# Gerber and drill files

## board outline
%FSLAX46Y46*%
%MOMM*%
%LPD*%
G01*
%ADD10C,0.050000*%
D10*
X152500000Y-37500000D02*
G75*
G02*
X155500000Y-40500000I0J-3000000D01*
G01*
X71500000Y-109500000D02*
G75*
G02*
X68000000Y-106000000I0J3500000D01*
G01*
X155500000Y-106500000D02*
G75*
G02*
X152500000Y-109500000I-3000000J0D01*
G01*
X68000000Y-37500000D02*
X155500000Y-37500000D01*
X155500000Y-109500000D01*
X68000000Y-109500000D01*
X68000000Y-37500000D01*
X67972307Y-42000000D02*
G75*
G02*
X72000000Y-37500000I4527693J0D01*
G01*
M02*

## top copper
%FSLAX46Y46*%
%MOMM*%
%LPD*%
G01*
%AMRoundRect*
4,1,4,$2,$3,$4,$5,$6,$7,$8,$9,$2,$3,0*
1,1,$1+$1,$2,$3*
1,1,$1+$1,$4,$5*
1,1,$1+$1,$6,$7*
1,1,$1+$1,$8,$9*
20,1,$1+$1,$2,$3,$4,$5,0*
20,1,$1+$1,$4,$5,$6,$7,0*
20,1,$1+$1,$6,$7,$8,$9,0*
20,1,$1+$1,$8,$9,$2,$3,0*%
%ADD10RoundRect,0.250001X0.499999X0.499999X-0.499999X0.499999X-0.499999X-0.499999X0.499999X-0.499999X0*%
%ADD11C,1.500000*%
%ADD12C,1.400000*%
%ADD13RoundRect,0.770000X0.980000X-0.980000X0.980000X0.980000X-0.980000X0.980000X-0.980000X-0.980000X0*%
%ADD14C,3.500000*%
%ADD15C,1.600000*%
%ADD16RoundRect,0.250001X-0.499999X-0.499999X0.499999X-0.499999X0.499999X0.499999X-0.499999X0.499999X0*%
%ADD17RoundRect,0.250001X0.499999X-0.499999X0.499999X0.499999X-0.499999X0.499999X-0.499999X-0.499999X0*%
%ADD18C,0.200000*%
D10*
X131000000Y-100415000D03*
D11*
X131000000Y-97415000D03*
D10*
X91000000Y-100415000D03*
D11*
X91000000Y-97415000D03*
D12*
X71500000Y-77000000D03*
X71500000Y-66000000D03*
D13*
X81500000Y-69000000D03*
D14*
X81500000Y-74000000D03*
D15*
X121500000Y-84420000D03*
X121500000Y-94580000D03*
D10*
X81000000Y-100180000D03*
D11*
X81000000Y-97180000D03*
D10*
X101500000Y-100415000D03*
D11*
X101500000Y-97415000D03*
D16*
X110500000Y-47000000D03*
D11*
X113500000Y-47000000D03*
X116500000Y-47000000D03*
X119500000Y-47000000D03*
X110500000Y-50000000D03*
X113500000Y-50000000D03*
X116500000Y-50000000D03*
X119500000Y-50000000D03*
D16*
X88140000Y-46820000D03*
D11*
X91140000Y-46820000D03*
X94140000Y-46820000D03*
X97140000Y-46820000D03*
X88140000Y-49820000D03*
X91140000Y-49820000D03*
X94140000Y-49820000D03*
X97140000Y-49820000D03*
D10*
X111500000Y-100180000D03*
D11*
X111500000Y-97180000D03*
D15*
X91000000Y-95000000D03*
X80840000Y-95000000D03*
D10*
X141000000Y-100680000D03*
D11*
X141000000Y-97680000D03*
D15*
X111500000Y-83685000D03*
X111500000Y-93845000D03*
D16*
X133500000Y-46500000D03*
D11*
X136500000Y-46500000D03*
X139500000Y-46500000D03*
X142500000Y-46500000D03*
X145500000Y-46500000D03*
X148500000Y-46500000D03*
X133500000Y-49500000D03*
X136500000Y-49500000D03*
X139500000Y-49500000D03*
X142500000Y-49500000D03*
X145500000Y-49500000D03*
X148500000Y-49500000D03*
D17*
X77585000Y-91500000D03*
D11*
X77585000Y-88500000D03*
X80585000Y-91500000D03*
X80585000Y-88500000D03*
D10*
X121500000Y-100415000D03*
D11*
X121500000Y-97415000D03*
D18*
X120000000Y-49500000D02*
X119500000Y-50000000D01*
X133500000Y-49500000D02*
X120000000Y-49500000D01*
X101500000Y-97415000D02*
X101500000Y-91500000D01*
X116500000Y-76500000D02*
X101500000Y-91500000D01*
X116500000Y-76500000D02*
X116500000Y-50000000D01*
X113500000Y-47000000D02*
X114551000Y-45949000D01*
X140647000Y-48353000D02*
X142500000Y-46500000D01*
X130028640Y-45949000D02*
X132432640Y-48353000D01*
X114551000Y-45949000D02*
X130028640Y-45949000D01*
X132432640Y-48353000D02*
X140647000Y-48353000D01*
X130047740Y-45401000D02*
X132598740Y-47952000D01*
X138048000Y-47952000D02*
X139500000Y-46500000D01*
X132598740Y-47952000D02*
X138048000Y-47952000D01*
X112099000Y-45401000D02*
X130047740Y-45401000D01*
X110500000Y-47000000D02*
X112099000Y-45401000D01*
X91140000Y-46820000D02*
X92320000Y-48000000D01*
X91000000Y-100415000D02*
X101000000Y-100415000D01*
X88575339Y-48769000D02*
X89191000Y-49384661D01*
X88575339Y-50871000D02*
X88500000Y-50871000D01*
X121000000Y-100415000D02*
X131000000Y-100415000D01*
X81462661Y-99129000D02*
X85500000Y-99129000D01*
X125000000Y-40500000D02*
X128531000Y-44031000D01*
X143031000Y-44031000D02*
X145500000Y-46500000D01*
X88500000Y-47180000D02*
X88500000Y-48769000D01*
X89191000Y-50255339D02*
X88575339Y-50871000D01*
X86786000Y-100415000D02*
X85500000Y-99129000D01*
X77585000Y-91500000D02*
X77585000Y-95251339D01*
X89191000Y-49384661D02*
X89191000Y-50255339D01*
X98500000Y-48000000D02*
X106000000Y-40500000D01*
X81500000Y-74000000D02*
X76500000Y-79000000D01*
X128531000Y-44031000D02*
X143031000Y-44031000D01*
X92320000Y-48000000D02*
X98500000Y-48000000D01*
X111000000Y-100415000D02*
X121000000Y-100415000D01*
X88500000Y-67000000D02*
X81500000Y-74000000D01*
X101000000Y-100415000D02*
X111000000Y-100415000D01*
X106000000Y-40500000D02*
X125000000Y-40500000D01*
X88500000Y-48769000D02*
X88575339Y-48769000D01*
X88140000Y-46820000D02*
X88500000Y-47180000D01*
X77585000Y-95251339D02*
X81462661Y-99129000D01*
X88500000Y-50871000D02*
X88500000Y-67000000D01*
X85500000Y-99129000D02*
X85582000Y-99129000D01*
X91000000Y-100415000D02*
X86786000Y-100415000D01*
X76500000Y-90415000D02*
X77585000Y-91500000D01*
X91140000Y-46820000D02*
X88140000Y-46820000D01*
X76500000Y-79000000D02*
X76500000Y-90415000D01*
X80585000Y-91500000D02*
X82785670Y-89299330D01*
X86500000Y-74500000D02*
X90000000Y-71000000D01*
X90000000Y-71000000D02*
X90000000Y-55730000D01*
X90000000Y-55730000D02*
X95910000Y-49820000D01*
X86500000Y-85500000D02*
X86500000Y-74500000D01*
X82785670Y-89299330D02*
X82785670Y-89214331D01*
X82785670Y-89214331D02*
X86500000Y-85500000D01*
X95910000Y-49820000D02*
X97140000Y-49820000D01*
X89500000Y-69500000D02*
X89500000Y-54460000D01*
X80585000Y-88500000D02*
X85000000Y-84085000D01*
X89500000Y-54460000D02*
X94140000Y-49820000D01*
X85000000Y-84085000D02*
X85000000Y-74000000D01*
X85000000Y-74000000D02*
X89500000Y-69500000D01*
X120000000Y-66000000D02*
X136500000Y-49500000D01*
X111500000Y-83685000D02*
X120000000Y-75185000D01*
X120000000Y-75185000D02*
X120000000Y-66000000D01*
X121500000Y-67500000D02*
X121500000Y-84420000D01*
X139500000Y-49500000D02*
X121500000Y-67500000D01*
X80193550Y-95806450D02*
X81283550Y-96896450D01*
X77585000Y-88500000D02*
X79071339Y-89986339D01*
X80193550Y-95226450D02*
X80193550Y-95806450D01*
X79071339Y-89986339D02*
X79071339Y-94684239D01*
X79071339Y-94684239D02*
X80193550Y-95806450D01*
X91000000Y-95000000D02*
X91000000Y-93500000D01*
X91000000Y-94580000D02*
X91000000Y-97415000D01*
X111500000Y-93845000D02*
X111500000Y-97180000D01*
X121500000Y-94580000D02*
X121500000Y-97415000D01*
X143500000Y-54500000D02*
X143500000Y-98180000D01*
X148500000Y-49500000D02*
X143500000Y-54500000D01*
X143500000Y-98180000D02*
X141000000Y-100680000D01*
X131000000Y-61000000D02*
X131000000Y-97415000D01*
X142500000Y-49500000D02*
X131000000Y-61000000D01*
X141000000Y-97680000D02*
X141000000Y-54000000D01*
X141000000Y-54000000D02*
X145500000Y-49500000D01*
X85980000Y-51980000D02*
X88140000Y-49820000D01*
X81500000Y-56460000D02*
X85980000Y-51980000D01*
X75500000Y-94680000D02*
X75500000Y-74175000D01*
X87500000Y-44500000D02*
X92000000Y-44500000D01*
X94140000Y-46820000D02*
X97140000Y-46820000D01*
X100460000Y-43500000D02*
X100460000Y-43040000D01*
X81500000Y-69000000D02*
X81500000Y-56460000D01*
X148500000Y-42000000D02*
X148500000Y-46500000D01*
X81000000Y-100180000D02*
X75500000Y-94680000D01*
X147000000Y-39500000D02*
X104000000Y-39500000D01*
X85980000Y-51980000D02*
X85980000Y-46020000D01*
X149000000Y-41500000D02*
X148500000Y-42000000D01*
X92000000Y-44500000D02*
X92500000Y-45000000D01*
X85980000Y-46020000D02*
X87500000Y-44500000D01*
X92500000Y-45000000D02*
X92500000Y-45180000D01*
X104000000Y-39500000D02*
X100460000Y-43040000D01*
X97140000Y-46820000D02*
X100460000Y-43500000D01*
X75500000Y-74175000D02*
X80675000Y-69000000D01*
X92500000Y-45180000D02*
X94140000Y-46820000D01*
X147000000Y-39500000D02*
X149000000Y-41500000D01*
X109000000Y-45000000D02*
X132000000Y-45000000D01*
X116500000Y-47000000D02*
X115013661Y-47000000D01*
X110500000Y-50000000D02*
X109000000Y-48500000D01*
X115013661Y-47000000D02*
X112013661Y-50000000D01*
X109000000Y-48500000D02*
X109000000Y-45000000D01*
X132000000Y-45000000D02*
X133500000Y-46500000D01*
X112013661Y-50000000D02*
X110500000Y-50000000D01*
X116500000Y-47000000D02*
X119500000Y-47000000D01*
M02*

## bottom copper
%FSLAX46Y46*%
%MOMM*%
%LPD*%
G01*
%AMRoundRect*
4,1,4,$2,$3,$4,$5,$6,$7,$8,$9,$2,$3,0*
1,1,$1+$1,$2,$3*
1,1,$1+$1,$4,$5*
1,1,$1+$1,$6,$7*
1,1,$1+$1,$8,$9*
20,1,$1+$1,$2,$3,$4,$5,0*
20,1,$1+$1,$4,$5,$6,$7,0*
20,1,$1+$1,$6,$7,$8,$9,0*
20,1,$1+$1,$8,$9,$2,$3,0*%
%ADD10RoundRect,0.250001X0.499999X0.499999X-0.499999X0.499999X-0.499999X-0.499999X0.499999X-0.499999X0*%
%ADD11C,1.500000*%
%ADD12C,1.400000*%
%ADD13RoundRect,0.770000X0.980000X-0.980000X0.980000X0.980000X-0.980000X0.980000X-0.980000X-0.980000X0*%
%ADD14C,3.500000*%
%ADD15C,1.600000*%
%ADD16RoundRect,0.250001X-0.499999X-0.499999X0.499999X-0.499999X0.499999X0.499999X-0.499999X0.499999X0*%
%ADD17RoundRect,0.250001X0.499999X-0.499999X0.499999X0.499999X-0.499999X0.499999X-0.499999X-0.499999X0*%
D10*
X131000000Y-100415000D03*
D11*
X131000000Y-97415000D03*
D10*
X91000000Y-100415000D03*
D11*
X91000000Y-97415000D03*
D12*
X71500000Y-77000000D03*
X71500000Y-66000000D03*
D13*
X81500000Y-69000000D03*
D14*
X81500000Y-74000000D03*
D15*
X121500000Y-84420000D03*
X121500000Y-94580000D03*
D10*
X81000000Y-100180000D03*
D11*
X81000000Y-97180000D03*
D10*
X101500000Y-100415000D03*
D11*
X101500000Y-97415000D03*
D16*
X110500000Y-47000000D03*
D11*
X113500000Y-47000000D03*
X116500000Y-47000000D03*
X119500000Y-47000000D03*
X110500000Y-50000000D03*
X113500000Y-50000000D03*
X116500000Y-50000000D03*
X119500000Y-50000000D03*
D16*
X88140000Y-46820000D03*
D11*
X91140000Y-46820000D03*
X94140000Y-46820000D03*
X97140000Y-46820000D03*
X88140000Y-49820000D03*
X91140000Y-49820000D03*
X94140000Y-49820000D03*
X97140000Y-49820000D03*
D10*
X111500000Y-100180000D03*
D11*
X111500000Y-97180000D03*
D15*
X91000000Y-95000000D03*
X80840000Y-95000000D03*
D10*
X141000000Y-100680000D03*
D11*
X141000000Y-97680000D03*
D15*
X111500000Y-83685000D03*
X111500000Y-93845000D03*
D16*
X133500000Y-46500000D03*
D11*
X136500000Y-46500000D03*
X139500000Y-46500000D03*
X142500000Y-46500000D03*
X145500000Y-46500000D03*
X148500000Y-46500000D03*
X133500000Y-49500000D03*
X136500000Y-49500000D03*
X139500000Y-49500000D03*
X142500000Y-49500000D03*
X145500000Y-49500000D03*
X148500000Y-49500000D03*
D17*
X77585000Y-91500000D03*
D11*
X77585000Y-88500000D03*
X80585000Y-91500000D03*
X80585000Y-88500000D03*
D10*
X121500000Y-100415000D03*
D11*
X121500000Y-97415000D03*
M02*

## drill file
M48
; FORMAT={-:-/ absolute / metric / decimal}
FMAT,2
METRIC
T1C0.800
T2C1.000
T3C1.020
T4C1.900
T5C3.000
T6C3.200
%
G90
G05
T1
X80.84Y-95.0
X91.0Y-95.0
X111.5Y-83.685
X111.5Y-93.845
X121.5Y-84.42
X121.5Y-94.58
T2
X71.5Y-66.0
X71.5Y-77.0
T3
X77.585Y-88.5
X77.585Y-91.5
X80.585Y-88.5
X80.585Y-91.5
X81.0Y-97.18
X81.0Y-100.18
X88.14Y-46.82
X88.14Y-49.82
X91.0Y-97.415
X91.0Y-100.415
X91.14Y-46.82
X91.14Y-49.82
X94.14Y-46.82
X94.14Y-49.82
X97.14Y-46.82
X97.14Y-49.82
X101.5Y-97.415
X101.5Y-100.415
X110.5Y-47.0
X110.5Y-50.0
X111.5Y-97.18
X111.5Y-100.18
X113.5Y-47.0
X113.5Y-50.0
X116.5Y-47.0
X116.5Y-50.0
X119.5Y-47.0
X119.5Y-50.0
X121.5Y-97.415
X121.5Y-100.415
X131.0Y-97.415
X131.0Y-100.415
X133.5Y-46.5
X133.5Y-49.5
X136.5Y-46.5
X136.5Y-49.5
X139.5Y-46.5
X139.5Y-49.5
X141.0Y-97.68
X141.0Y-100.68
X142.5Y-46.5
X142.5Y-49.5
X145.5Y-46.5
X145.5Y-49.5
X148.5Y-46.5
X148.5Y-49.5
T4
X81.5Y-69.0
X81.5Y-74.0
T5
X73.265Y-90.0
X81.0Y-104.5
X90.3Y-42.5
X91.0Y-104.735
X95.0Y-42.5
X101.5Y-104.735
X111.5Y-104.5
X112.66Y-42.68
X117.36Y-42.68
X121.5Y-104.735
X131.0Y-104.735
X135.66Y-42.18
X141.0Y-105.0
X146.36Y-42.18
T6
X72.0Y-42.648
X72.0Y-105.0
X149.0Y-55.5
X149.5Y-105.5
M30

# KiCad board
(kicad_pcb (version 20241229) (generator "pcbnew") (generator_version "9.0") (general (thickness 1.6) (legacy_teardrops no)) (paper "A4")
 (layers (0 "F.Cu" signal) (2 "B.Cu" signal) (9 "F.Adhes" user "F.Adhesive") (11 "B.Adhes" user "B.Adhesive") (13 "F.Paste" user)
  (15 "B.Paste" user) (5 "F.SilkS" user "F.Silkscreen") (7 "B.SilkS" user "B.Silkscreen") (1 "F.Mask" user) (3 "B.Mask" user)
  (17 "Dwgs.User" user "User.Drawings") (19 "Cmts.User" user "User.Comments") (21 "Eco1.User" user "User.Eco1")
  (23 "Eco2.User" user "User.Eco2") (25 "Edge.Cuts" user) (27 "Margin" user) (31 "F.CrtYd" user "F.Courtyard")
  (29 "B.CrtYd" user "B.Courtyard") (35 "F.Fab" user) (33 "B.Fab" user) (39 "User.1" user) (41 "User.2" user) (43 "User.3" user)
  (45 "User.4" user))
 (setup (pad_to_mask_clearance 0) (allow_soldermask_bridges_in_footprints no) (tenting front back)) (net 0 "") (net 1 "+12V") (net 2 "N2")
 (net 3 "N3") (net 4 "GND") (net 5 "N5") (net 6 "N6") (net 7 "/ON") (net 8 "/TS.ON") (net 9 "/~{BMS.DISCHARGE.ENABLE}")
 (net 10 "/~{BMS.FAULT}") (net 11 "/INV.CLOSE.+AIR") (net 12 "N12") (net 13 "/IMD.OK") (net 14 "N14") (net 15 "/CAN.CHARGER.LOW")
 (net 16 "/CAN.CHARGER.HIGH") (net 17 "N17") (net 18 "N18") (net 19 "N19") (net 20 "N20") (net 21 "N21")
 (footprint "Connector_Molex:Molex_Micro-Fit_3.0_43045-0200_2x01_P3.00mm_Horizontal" (layer "F.Cu") (at 131 100.415 180)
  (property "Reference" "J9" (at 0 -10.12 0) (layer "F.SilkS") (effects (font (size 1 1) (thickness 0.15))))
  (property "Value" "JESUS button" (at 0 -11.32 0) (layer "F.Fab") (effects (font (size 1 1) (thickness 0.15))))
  (pad "" np_thru_hole circle (at 0 -4.32 180) (size 3 3) (drill 3) (layers "*.Cu" "*.Mask"))
  (pad "1" thru_hole roundrect (at 0 0 180) (size 1.5 1.5) (drill 1.02) (layers "*.Cu" "*.Mask") (remove_unused_layers no)
   (roundrect_rratio 0.166667) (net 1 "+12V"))
  (pad "2" thru_hole circle (at 0 3 180) (size 1.5 1.5) (drill 1.02) (layers "*.Cu" "*.Mask") (remove_unused_layers no) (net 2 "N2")))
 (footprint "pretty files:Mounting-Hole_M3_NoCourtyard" (layer "F.Cu") (at 150.41 110.58)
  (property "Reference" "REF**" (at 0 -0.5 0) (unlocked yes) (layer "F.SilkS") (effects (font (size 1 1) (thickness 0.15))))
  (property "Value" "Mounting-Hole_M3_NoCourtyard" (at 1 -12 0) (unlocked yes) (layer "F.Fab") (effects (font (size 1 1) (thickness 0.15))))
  (pad "" np_thru_hole circle (at -0.91 -5.08) (size 3.2 3.2) (drill 3.2) (layers "*.Cu" "*.Mask")))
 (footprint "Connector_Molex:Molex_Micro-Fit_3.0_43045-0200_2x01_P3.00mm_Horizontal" (layer "F.Cu") (at 91 100.415 180)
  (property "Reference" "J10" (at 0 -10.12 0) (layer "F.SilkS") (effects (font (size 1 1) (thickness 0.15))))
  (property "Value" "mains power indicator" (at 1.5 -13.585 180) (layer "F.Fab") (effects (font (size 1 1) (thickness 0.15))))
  (pad "" np_thru_hole circle (at 0 -4.32 180) (size 3 3) (drill 3) (layers "*.Cu" "*.Mask"))
  (pad "1" thru_hole roundrect (at 0 0 180) (size 1.5 1.5) (drill 1.02) (layers "*.Cu" "*.Mask") (remove_unused_layers no)
   (roundrect_rratio 0.166667) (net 1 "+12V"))
  (pad "2" thru_hole circle (at 0 3 180) (size 1.5 1.5) (drill 1.02) (layers "*.Cu" "*.Mask") (remove_unused_layers no) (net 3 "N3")))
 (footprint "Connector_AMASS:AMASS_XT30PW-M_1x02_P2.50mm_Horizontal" (layer "F.Cu") (at 81.5 69 90)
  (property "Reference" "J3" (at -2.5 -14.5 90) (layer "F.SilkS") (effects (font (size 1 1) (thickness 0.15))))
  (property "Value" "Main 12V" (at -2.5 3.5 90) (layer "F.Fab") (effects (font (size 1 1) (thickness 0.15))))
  (pad "" thru_hole circle (at -8 -10 90) (size 1.4 1.4) (drill 1) (layers "*.Cu" "*.Mask") (remove_unused_layers no))
  (pad "" thru_hole circle (at 3 -10 90) (size 1.4 1.4) (drill 1) (layers "*.Cu" "*.Mask") (remove_unused_layers no))
  (pad "1" thru_hole roundrect (at 0 0 90) (size 3.5 3.5) (drill 1.9) (layers "*.Cu" "*.Mask") (remove_unused_layers no)
   (roundrect_rratio 0.22) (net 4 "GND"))
  (pad "2" thru_hole circle (at -5 0 90) (size 3.5 3.5) (drill 1.9) (layers "*.Cu" "*.Mask") (remove_unused_layers no) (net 1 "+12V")))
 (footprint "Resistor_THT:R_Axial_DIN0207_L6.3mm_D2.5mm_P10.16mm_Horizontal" (layer "F.Cu") (at 121.5 84.42 -90)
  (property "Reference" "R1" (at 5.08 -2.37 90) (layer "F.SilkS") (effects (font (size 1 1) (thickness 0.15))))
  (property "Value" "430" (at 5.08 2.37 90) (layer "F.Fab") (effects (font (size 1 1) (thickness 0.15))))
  (pad "1" thru_hole circle (at 0 0 270) (size 1.6 1.6) (drill 0.8) (layers "*.Cu" "*.Mask") (remove_unused_layers no) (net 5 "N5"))
  (pad "2" thru_hole circle (at 10.16 0 270) (size 1.6 1.6) (drill 0.8) (layers "*.Cu" "*.Mask") (remove_unused_layers no) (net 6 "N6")))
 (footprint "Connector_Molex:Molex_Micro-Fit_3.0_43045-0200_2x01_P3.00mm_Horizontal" (layer "F.Cu") (at 81 100.18 180)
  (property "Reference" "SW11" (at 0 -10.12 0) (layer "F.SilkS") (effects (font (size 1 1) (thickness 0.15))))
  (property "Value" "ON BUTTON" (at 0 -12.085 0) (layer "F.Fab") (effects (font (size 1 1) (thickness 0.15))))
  (pad "" np_thru_hole circle (at 0 -4.32 180) (size 3 3) (drill 3) (layers "*.Cu" "*.Mask"))
  (pad "1" thru_hole roundrect (at 0 0 180) (size 1.5 1.5) (drill 1.02) (layers "*.Cu" "*.Mask") (remove_unused_layers no)
   (roundrect_rratio 0.166667) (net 4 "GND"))
  (pad "2" thru_hole circle (at 0 3 180) (size 1.5 1.5) (drill 1.02) (layers "*.Cu" "*.Mask") (remove_unused_layers no) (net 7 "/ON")))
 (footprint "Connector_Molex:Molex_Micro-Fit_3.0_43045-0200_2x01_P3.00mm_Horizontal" (layer "F.Cu") (at 101.5 100.415 180)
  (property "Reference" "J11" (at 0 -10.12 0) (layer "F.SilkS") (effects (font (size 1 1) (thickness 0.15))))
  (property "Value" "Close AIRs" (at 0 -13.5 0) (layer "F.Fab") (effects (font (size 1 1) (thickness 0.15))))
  (pad "" np_thru_hole circle (at 0 -4.32 180) (size 3 3) (drill 3) (layers "*.Cu" "*.Mask"))
  (pad "1" thru_hole roundrect (at 0 0 180) (size 1.5 1.5) (drill 1.02) (layers "*.Cu" "*.Mask") (remove_unused_layers no)
   (roundrect_rratio 0.166667) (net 1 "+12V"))
  (pad "2" thru_hole circle (at 0 3 180) (size 1.5 1.5) (drill 1.02) (layers "*.Cu" "*.Mask") (remove_unused_layers no) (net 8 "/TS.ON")))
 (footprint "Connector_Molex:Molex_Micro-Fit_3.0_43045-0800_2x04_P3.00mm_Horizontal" (layer "F.Cu") (at 110.5 47)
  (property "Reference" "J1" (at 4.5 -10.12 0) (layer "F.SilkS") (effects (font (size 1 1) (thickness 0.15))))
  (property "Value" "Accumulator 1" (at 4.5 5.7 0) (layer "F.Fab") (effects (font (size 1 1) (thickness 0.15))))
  (pad "" np_thru_hole circle (at 2.16 -4.32) (size 3 3) (drill 3) (layers "*.Cu" "*.Mask"))
  (pad "" np_thru_hole circle (at 6.86 -4.32) (size 3 3) (drill 3) (layers "*.Cu" "*.Mask"))
  (pad "1" thru_hole roundrect (at 0 0) (size 1.5 1.5) (drill 1.02) (layers "*.Cu" "*.Mask") (remove_unused_layers no)
   (roundrect_rratio 0.166667) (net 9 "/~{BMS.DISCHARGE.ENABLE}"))
  (pad "2" thru_hole circle (at 3 0) (size 1.5 1.5) (drill 1.02) (layers "*.Cu" "*.Mask") (remove_unused_layers no) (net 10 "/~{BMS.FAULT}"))
  (pad "3" thru_hole circle (at 6 0) (size 1.5 1.5) (drill 1.02) (layers "*.Cu" "*.Mask") (remove_unused_layers no)
   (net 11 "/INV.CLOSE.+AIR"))
  (pad "4" thru_hole circle (at 9 0) (size 1.5 1.5) (drill 1.02) (layers "*.Cu" "*.Mask") (remove_unused_layers no)
   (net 11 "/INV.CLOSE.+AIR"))
  (pad "5" thru_hole circle (at 0 3) (size 1.5 1.5) (drill 1.02) (layers "*.Cu" "*.Mask") (remove_unused_layers no)
   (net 11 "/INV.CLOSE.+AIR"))
  (pad "6" thru_hole circle (at 3 3) (size 1.5 1.5) (drill 1.02) (layers "*.Cu" "*.Mask") (remove_unused_layers no) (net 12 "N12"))
  (pad "7" thru_hole circle (at 6 3) (size 1.5 1.5) (drill 1.02) (layers "*.Cu" "*.Mask") (remove_unused_layers no) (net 8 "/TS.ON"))
  (pad "8" thru_hole circle (at 9 3) (size 1.5 1.5) (drill 1.02) (layers "*.Cu" "*.Mask") (remove_unused_layers no) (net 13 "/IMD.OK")))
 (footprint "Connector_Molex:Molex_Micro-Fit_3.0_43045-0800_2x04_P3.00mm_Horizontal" (layer "F.Cu") (at 88.14 46.82)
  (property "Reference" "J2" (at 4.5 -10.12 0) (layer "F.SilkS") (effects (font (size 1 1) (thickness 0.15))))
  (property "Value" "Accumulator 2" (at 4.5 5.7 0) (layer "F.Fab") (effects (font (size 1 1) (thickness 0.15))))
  (pad "" np_thru_hole circle (at 2.16 -4.32) (size 3 3) (drill 3) (layers "*.Cu" "*.Mask"))
  (pad "" np_thru_hole circle (at 6.86 -4.32) (size 3 3) (drill 3) (layers "*.Cu" "*.Mask"))
  (pad "1" thru_hole roundrect (at 0 0) (size 1.5 1.5) (drill 1.02) (layers "*.Cu" "*.Mask") (remove_unused_layers no)
   (roundrect_rratio 0.166667) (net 1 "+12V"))
  (pad "2" thru_hole circle (at 3 0) (size 1.5 1.5) (drill 1.02) (layers "*.Cu" "*.Mask") (remove_unused_layers no) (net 1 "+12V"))
  (pad "3" thru_hole circle (at 6 0) (size 1.5 1.5) (drill 1.02) (layers "*.Cu" "*.Mask") (remove_unused_layers no) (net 4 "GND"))
  (pad "4" thru_hole circle (at 9 0) (size 1.5 1.5) (drill 1.02) (layers "*.Cu" "*.Mask") (remove_unused_layers no) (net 4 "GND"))
  (pad "5" thru_hole circle (at 0 3) (size 1.5 1.5) (drill 1.02) (layers "*.Cu" "*.Mask") (remove_unused_layers no) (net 4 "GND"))
  (pad "6" thru_hole circle (at 3 3) (size 1.5 1.5) (drill 1.02) (layers "*.Cu" "*.Mask") (remove_unused_layers no) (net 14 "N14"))
  (pad "7" thru_hole circle (at 6 3) (size 1.5 1.5) (drill 1.02) (layers "*.Cu" "*.Mask") (remove_unused_layers no)
   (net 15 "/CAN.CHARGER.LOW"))
  (pad "8" thru_hole circle (at 9 3) (size 1.5 1.5) (drill 1.02) (layers "*.Cu" "*.Mask") (remove_unused_layers no)
   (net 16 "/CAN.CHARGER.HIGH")))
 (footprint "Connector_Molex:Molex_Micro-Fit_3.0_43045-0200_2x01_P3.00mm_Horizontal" (layer "F.Cu") (at 111.5 100.18 180)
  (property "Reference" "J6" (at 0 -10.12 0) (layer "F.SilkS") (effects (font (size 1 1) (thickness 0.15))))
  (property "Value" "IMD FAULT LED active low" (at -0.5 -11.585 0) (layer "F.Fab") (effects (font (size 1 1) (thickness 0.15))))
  (pad "" np_thru_hole circle (at 0 -4.32 180) (size 3 3) (drill 3) (layers "*.Cu" "*.Mask"))
  (pad "1" thru_hole roundrect (at 0 0 180) (size 1.5 1.5) (drill 1.02) (layers "*.Cu" "*.Mask") (remove_unused_layers no)
   (roundrect_rratio 0.166667) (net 1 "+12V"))
  (pad "2" thru_hole circle (at 0 3 180) (size 1.5 1.5) (drill 1.02) (layers "*.Cu" "*.Mask") (remove_unused_layers no) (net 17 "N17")))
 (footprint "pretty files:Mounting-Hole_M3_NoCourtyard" (layer "F.Cu") (at 149.91 60.58)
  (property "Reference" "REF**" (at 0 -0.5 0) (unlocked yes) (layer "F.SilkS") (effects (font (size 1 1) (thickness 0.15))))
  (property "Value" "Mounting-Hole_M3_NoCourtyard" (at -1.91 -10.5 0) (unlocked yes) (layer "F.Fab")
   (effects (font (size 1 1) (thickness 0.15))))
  (pad "" np_thru_hole circle (at -0.91 -5.08) (size 3.2 3.2) (drill 3.2) (layers "*.Cu" "*.Mask")))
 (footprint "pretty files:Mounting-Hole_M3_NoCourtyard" (layer "F.Cu") (at 72.91 47.7275)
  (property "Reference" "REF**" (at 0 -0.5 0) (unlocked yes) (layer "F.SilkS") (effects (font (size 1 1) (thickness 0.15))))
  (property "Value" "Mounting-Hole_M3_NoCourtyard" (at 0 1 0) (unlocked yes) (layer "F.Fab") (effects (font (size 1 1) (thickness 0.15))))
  (pad "" np_thru_hole circle (at -0.91 -5.08) (size 3.2 3.2) (drill 3.2) (layers "*.Cu" "*.Mask")))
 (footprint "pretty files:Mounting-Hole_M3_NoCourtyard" (layer "F.Cu") (at 72.91 110.08)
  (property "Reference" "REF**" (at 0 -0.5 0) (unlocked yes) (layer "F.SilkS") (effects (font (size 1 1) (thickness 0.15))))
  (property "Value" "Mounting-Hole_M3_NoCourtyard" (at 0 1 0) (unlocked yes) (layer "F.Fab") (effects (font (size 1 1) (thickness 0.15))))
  (pad "" np_thru_hole circle (at -0.91 -5.08) (size 3.2 3.2) (drill 3.2) (layers "*.Cu" "*.Mask")))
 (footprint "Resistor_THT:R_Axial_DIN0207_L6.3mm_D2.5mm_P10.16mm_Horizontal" (layer "F.Cu") (at 91 95 180)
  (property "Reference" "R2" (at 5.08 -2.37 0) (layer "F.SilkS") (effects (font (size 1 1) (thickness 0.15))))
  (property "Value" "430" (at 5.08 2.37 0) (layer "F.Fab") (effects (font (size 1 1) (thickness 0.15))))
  (pad "1" thru_hole circle (at 0 0 180) (size 1.6 1.6) (drill 0.8) (layers "*.Cu" "*.Mask") (remove_unused_layers no) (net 3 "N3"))
  (pad "2" thru_hole circle (at 10.16 0 180) (size 1.6 1.6) (drill 0.8) (layers "*.Cu" "*.Mask") (remove_unused_layers no) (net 7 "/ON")))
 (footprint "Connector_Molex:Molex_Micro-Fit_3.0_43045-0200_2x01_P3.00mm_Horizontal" (layer "F.Cu") (at 141 100.68 180)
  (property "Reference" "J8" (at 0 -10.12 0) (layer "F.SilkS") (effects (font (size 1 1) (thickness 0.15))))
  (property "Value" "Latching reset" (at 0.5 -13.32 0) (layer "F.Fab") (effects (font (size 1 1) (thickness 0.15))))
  (pad "" np_thru_hole circle (at 0 -4.32 180) (size 3 3) (drill 3) (layers "*.Cu" "*.Mask"))
  (pad "1" thru_hole roundrect (at 0 0 180) (size 1.5 1.5) (drill 1.02) (layers "*.Cu" "*.Mask") (remove_unused_layers no)
   (roundrect_rratio 0.166667) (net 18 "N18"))
  (pad "2" thru_hole circle (at 0 3 180) (size 1.5 1.5) (drill 1.02) (layers "*.Cu" "*.Mask") (remove_unused_layers no) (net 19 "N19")))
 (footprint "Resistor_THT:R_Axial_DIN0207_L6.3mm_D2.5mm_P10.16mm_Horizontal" (layer "F.Cu") (at 111.5 83.685 -90)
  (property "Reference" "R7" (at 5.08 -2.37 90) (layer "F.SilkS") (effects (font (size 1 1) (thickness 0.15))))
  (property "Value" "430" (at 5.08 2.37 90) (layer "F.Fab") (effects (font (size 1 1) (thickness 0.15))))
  (pad "1" thru_hole circle (at 0 0 270) (size 1.6 1.6) (drill 0.8) (layers "*.Cu" "*.Mask") (remove_unused_layers no) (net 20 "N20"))
  (pad "2" thru_hole circle (at 10.16 0 270) (size 1.6 1.6) (drill 0.8) (layers "*.Cu" "*.Mask") (remove_unused_layers no) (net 17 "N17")))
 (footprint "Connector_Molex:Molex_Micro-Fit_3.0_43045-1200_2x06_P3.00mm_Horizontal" (layer "F.Cu") (at 133.5 46.5)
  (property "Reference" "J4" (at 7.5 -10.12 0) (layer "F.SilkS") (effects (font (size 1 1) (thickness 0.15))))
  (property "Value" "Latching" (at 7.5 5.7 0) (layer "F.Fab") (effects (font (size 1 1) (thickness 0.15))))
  (pad "" np_thru_hole circle (at 2.16 -4.32) (size 3 3) (drill 3) (layers "*.Cu" "*.Mask"))
  (pad "" np_thru_hole circle (at 12.86 -4.32) (size 3 3) (drill 3) (layers "*.Cu" "*.Mask"))
  (pad "1" thru_hole roundrect (at 0 0) (size 1.5 1.5) (drill 1.02) (layers "*.Cu" "*.Mask") (remove_unused_layers no)
   (roundrect_rratio 0.166667) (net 11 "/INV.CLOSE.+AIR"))
  (pad "2" thru_hole circle (at 3 0) (size 1.5 1.5) (drill 1.02) (layers "*.Cu" "*.Mask") (remove_unused_layers no) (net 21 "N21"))
  (pad "3" thru_hole circle (at 6 0) (size 1.5 1.5) (drill 1.02) (layers "*.Cu" "*.Mask") (remove_unused_layers no)
   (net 9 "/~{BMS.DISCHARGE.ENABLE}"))
  (pad "4" thru_hole circle (at 9 0) (size 1.5 1.5) (drill 1.02) (layers "*.Cu" "*.Mask") (remove_unused_layers no) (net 10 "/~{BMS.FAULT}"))
  (pad "5" thru_hole circle (at 12 0) (size 1.5 1.5) (drill 1.02) (layers "*.Cu" "*.Mask") (remove_unused_layers no) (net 1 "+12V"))
  (pad "6" thru_hole circle (at 15 0) (size 1.5 1.5) (drill 1.02) (layers "*.Cu" "*.Mask") (remove_unused_layers no) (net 4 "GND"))
  (pad "7" thru_hole circle (at 0 3) (size 1.5 1.5) (drill 1.02) (layers "*.Cu" "*.Mask") (remove_unused_layers no) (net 13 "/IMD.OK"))
  (pad "8" thru_hole circle (at 3 3) (size 1.5 1.5) (drill 1.02) (layers "*.Cu" "*.Mask") (remove_unused_layers no) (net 20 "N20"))
  (pad "9" thru_hole circle (at 6 3) (size 1.5 1.5) (drill 1.02) (layers "*.Cu" "*.Mask") (remove_unused_layers no) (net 5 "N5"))
  (pad "10" thru_hole circle (at 9 3) (size 1.5 1.5) (drill 1.02) (layers "*.Cu" "*.Mask") (remove_unused_layers no) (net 2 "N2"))
  (pad "11" thru_hole circle (at 12 3) (size 1.5 1.5) (drill 1.02) (layers "*.Cu" "*.Mask") (remove_unused_layers no) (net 19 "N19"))
  (pad "12" thru_hole circle (at 15 3) (size 1.5 1.5) (drill 1.02) (layers "*.Cu" "*.Mask") (remove_unused_layers no) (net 18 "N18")))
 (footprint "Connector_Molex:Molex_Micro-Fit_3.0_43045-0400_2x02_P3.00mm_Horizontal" (layer "F.Cu") (at 77.585 91.5 90)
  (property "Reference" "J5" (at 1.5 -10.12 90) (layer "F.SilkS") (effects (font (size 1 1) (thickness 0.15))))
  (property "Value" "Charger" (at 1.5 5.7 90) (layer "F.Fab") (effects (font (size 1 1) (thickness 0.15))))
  (pad "" np_thru_hole circle (at 1.5 -4.32 90) (size 3 3) (drill 3) (layers "*.Cu" "*.Mask"))
  (pad "1" thru_hole roundrect (at 0 0 90) (size 1.5 1.5) (drill 1.02) (layers "*.Cu" "*.Mask") (remove_unused_layers no)
   (roundrect_rratio 0.166667) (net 1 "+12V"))
  (pad "2" thru_hole circle (at 3 0 90) (size 1.5 1.5) (drill 1.02) (layers "*.Cu" "*.Mask") (remove_unused_layers no) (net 7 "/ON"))
  (pad "3" thru_hole circle (at 0 3 90) (size 1.5 1.5) (drill 1.02) (layers "*.Cu" "*.Mask") (remove_unused_layers no)
   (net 16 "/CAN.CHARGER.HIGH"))
  (pad "4" thru_hole circle (at 3 3 90) (size 1.5 1.5) (drill 1.02) (layers "*.Cu" "*.Mask") (remove_unused_layers no)
   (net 15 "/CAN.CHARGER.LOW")))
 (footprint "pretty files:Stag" (layer "F.Cu") (at 132 74.5)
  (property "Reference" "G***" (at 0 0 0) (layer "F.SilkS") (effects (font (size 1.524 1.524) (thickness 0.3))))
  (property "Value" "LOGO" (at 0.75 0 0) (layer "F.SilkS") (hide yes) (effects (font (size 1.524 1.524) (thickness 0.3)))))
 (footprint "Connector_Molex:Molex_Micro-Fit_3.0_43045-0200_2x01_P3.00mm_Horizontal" (layer "F.Cu") (at 121.5 100.415 180)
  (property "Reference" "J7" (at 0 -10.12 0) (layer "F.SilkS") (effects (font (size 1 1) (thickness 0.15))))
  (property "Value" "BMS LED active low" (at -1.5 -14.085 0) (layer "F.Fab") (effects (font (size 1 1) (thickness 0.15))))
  (pad "" np_thru_hole circle (at 0 -4.32 180) (size 3 3) (drill 3) (layers "*.Cu" "*.Mask"))
  (pad "1" thru_hole roundrect (at 0 0 180) (size 1.5 1.5) (drill 1.02) (layers "*.Cu" "*.Mask") (remove_unused_layers no)
   (roundrect_rratio 0.166667) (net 1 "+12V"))
  (pad "2" thru_hole circle (at 0 3 180) (size 1.5 1.5) (drill 1.02) (layers "*.Cu" "*.Mask") (remove_unused_layers no) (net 6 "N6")))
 (gr_arc (start 152.5 37.5) (mid 154.62132 38.37868) (end 155.5 40.5) (stroke (width 0.05) (type default)) (layer "Edge.Cuts"))
 (gr_arc (start 71.5 109.5) (mid 69.025126 108.474874) (end 68 106) (stroke (width 0.05) (type default)) (layer "Edge.Cuts"))
 (gr_arc (start 155.5 106.5) (mid 154.62132 108.62132) (end 152.5 109.5) (stroke (width 0.05) (type default)) (layer "Edge.Cuts"))
 (gr_rect (start 68 37.5) (end 155.5 109.5) (stroke (width 0.05) (type default)) (fill no) (layer "Edge.Cuts"))
 (gr_arc (start 67.972307 42) (mid 69.126289 38.980384) (end 72 37.5) (stroke (width 0.05) (type default)) (layer "Edge.Cuts"))
 (segment (start 120 49.5) (end 119.5 50) (width 0.2) (layer "F.Cu") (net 13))
 (segment (start 133.5 49.5) (end 120 49.5) (width 0.2) (layer "F.Cu") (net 13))
 (segment (start 101.5 97.415) (end 101.5 91.5) (width 0.2) (layer "F.Cu") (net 8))
 (segment (start 116.5 76.5) (end 101.5 91.5) (width 0.2) (layer "F.Cu") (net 8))
 (segment (start 116.5 76.5) (end 116.5 50) (width 0.2) (layer "F.Cu") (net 8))
 (segment (start 113.5 47) (end 114.551 45.949) (width 0.2) (layer "F.Cu") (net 10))
 (segment (start 140.647 48.353) (end 142.5 46.5) (width 0.2) (layer "F.Cu") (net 10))
 (segment (start 130.02864 45.949) (end 132.43264 48.353) (width 0.2) (layer "F.Cu") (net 10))
 (segment (start 114.551 45.949) (end 130.02864 45.949) (width 0.2) (layer "F.Cu") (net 10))
 (segment (start 132.43264 48.353) (end 140.647 48.353) (width 0.2) (layer "F.Cu") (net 10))
 (segment (start 130.04774 45.401) (end 132.59874 47.952) (width 0.2) (layer "F.Cu") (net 9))
 (segment (start 138.048 47.952) (end 139.5 46.5) (width 0.2) (layer "F.Cu") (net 9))
 (segment (start 132.59874 47.952) (end 138.048 47.952) (width 0.2) (layer "F.Cu") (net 9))
 (segment (start 112.099 45.401) (end 130.04774 45.401) (width 0.2) (layer "F.Cu") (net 9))
 (segment (start 110.5 47) (end 112.099 45.401) (width 0.2) (layer "F.Cu") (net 9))
 (segment (start 91.14 46.82) (end 92.32 48) (width 0.2) (layer "F.Cu") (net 1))
 (segment (start 91 100.415) (end 101 100.415) (width 0.2) (layer "F.Cu") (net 1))
 (segment (start 88.575339 48.769) (end 89.191 49.384661) (width 0.2) (layer "F.Cu") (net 1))
 (segment (start 88.575339 50.871) (end 88.5 50.871) (width 0.2) (layer "F.Cu") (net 1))
 (segment (start 121 100.415) (end 131 100.415) (width 0.2) (layer "F.Cu") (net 1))
 (segment (start 81.462661 99.129) (end 85.5 99.129) (width 0.2) (layer "F.Cu") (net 1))
 (segment (start 125 40.5) (end 128.531 44.031) (width 0.2) (layer "F.Cu") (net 1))
 (segment (start 143.031 44.031) (end 145.5 46.5) (width 0.2) (layer "F.Cu") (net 1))
 (segment (start 88.5 47.18) (end 88.5 48.769) (width 0.2) (layer "F.Cu") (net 1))
 (segment (start 89.191 50.255339) (end 88.575339 50.871) (width 0.2) (layer "F.Cu") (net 1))
 (segment (start 86.786 100.415) (end 85.5 99.129) (width 0.2) (layer "F.Cu") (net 1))
 (segment (start 77.585 91.5) (end 77.585 95.251339) (width 0.2) (layer "F.Cu") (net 1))
 (segment (start 89.191 49.384661) (end 89.191 50.255339) (width 0.2) (layer "F.Cu") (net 1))
 (segment (start 98.5 48) (end 106 40.5) (width 0.2) (layer "F.Cu") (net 1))
 (segment (start 81.5 74) (end 76.5 79) (width 0.2) (layer "F.Cu") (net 1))
 (segment (start 128.531 44.031) (end 143.031 44.031) (width 0.2) (layer "F.Cu") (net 1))
 (segment (start 92.32 48) (end 98.5 48) (width 0.2) (layer "F.Cu") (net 1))
 (segment (start 111 100.415) (end 121 100.415) (width 0.2) (layer "F.Cu") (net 1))
 (segment (start 88.5 67) (end 81.5 74) (width 0.2) (layer "F.Cu") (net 1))
 (segment (start 101 100.415) (end 111 100.415) (width 0.2) (layer "F.Cu") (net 1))
 (segment (start 106 40.5) (end 125 40.5) (width 0.2) (layer "F.Cu") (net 1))
 (segment (start 88.5 48.769) (end 88.575339 48.769) (width 0.2) (layer "F.Cu") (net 1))
 (segment (start 88.14 46.82) (end 88.5 47.18) (width 0.2) (layer "F.Cu") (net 1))
 (segment (start 77.585 95.251339) (end 81.462661 99.129) (width 0.2) (layer "F.Cu") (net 1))
 (segment (start 88.5 50.871) (end 88.5 67) (width 0.2) (layer "F.Cu") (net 1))
 (segment (start 85.5 99.129) (end 85.582 99.129) (width 0.2) (layer "F.Cu") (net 1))
 (segment (start 91 100.415) (end 86.786 100.415) (width 0.2) (layer "F.Cu") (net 1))
 (segment (start 76.5 90.415) (end 77.585 91.5) (width 0.2) (layer "F.Cu") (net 1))
 (segment (start 91.14 46.82) (end 88.14 46.82) (width 0.2) (layer "F.Cu") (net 1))
 (segment (start 76.5 79) (end 76.5 90.415) (width 0.2) (layer "F.Cu") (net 1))
 (segment (start 80.585 91.5) (end 82.78567 89.29933) (width 0.2) (layer "F.Cu") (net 16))
 (segment (start 86.5 74.5) (end 90 71) (width 0.2) (layer "F.Cu") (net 16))
 (segment (start 90 71) (end 90 55.73) (width 0.2) (layer "F.Cu") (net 16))
 (segment (start 90 55.73) (end 95.91 49.82) (width 0.2) (layer "F.Cu") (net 16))
 (segment (start 86.5 85.5) (end 86.5 74.5) (width 0.2) (layer "F.Cu") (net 16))
 (segment (start 82.78567 89.29933) (end 82.78567 89.214331) (width 0.2) (layer "F.Cu") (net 16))
 (segment (start 82.78567 89.214331) (end 86.5 85.5) (width 0.2) (layer "F.Cu") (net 16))
 (segment (start 95.91 49.82) (end 97.14 49.82) (width 0.2) (layer "F.Cu") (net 16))
 (segment (start 89.5 69.5) (end 89.5 54.46) (width 0.2) (layer "F.Cu") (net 15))
 (segment (start 80.585 88.5) (end 85 84.085) (width 0.2) (layer "F.Cu") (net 15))
 (segment (start 89.5 54.46) (end 94.14 49.82) (width 0.2) (layer "F.Cu") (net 15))
 (segment (start 85 84.085) (end 85 74) (width 0.2) (layer "F.Cu") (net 15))
 (segment (start 85 74) (end 89.5 69.5) (width 0.2) (layer "F.Cu") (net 15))
 (segment (start 120 66) (end 136.5 49.5) (width 0.2) (layer "F.Cu") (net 20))
 (segment (start 111.5 83.685) (end 120 75.185) (width 0.2) (layer "F.Cu") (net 20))
 (segment (start 120 75.185) (end 120 66) (width 0.2) (layer "F.Cu") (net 20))
 (segment (start 121.5 67.5) (end 121.5 84.42) (width 0.2) (layer "F.Cu") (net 5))
 (segment (start 139.5 49.5) (end 121.5 67.5) (width 0.2) (layer "F.Cu") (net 5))
 (segment (start 80.19355 95.80645) (end 81.28355 96.89645) (width 0.2) (layer "F.Cu") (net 7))
 (segment (start 77.585 88.5) (end 79.071339 89.986339) (width 0.2) (layer "F.Cu") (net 7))
 (segment (start 80.19355 95.22645) (end 80.19355 95.80645) (width 0.2) (layer "F.Cu") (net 7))
 (segment (start 79.071339 89.986339) (end 79.071339 94.684239) (width 0.2) (layer "F.Cu") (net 7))
 (segment (start 79.071339 94.684239) (end 80.19355 95.80645) (width 0.2) (layer "F.Cu") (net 7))
 (segment (start 91 95) (end 91 93.5) (width 0.2) (layer "F.Cu") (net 3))
 (segment (start 91 94.58) (end 91 97.415) (width 0.2) (layer "F.Cu") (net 3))
 (segment (start 111.5 93.845) (end 111.5 97.18) (width 0.2) (layer "F.Cu") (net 17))
 (segment (start 121.5 94.58) (end 121.5 97.415) (width 0.2) (layer "F.Cu") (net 6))
 (segment (start 143.5 54.5) (end 143.5 98.18) (width 0.2) (layer "F.Cu") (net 18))
 (segment (start 148.5 49.5) (end 143.5 54.5) (width 0.2) (layer "F.Cu") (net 18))
 (segment (start 143.5 98.18) (end 141 100.68) (width 0.2) (layer "F.Cu") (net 18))
 (segment (start 131 61) (end 131 97.415) (width 0.2) (layer "F.Cu") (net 2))
 (segment (start 142.5 49.5) (end 131 61) (width 0.2) (layer "F.Cu") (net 2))
 (segment (start 141 97.68) (end 141 54) (width 0.2) (layer "F.Cu") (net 19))
 (segment (start 141 54) (end 145.5 49.5) (width 0.2) (layer "F.Cu") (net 19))
 (segment (start 85.98 51.98) (end 88.14 49.82) (width 0.2) (layer "F.Cu") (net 4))
 (segment (start 81.5 56.46) (end 85.98 51.98) (width 0.2) (layer "F.Cu") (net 4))
 (segment (start 75.5 94.68) (end 75.5 74.175) (width 0.2) (layer "F.Cu") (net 4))
 (segment (start 87.5 44.5) (end 92 44.5) (width 0.2) (layer "F.Cu") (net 4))
 (segment (start 94.14 46.82) (end 97.14 46.82) (width 0.2) (layer "F.Cu") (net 4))
 (segment (start 100.46 43.5) (end 100.46 43.04) (width 0.2) (layer "F.Cu") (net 4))
 (segment (start 81.5 69) (end 81.5 56.46) (width 0.2) (layer "F.Cu") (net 4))
 (segment (start 148.5 42) (end 148.5 46.5) (width 0.2) (layer "F.Cu") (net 4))
 (segment (start 81 100.18) (end 75.5 94.68) (width 0.2) (layer "F.Cu") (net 4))
 (segment (start 147 39.5) (end 104 39.5) (width 0.2) (layer "F.Cu") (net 4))
 (segment (start 85.98 51.98) (end 85.98 46.02) (width 0.2) (layer "F.Cu") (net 4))
 (segment (start 149 41.5) (end 148.5 42) (width 0.2) (layer "F.Cu") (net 4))
 (segment (start 92 44.5) (end 92.5 45) (width 0.2) (layer "F.Cu") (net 4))
 (segment (start 85.98 46.02) (end 87.5 44.5) (width 0.2) (layer "F.Cu") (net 4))
 (segment (start 92.5 45) (end 92.5 45.18) (width 0.2) (layer "F.Cu") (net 4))
 (segment (start 104 39.5) (end 100.46 43.04) (width 0.2) (layer "F.Cu") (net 4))
 (segment (start 97.14 46.82) (end 100.46 43.5) (width 0.2) (layer "F.Cu") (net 4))
 (segment (start 75.5 74.175) (end 80.675 69) (width 0.2) (layer "F.Cu") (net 4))
 (segment (start 92.5 45.18) (end 94.14 46.82) (width 0.2) (layer "F.Cu") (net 4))
 (segment (start 147 39.5) (end 149 41.5) (width 0.2) (layer "F.Cu") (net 4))
 (segment (start 109 45) (end 132 45) (width 0.2) (layer "F.Cu") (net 11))
 (segment (start 116.5 47) (end 115.013661 47) (width 0.2) (layer "F.Cu") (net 11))
 (segment (start 110.5 50) (end 109 48.5) (width 0.2) (layer "F.Cu") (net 11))
 (segment (start 115.013661 47) (end 112.013661 50) (width 0.2) (layer "F.Cu") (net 11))
 (segment (start 109 48.5) (end 109 45) (width 0.2) (layer "F.Cu") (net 11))
 (segment (start 132 45) (end 133.5 46.5) (width 0.2) (layer "F.Cu") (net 11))
 (segment (start 112.013661 50) (end 110.5 50) (width 0.2) (layer "F.Cu") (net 11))
 (segment (start 116.5 47) (end 119.5 47) (width 0.2) (layer "F.Cu") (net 11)))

